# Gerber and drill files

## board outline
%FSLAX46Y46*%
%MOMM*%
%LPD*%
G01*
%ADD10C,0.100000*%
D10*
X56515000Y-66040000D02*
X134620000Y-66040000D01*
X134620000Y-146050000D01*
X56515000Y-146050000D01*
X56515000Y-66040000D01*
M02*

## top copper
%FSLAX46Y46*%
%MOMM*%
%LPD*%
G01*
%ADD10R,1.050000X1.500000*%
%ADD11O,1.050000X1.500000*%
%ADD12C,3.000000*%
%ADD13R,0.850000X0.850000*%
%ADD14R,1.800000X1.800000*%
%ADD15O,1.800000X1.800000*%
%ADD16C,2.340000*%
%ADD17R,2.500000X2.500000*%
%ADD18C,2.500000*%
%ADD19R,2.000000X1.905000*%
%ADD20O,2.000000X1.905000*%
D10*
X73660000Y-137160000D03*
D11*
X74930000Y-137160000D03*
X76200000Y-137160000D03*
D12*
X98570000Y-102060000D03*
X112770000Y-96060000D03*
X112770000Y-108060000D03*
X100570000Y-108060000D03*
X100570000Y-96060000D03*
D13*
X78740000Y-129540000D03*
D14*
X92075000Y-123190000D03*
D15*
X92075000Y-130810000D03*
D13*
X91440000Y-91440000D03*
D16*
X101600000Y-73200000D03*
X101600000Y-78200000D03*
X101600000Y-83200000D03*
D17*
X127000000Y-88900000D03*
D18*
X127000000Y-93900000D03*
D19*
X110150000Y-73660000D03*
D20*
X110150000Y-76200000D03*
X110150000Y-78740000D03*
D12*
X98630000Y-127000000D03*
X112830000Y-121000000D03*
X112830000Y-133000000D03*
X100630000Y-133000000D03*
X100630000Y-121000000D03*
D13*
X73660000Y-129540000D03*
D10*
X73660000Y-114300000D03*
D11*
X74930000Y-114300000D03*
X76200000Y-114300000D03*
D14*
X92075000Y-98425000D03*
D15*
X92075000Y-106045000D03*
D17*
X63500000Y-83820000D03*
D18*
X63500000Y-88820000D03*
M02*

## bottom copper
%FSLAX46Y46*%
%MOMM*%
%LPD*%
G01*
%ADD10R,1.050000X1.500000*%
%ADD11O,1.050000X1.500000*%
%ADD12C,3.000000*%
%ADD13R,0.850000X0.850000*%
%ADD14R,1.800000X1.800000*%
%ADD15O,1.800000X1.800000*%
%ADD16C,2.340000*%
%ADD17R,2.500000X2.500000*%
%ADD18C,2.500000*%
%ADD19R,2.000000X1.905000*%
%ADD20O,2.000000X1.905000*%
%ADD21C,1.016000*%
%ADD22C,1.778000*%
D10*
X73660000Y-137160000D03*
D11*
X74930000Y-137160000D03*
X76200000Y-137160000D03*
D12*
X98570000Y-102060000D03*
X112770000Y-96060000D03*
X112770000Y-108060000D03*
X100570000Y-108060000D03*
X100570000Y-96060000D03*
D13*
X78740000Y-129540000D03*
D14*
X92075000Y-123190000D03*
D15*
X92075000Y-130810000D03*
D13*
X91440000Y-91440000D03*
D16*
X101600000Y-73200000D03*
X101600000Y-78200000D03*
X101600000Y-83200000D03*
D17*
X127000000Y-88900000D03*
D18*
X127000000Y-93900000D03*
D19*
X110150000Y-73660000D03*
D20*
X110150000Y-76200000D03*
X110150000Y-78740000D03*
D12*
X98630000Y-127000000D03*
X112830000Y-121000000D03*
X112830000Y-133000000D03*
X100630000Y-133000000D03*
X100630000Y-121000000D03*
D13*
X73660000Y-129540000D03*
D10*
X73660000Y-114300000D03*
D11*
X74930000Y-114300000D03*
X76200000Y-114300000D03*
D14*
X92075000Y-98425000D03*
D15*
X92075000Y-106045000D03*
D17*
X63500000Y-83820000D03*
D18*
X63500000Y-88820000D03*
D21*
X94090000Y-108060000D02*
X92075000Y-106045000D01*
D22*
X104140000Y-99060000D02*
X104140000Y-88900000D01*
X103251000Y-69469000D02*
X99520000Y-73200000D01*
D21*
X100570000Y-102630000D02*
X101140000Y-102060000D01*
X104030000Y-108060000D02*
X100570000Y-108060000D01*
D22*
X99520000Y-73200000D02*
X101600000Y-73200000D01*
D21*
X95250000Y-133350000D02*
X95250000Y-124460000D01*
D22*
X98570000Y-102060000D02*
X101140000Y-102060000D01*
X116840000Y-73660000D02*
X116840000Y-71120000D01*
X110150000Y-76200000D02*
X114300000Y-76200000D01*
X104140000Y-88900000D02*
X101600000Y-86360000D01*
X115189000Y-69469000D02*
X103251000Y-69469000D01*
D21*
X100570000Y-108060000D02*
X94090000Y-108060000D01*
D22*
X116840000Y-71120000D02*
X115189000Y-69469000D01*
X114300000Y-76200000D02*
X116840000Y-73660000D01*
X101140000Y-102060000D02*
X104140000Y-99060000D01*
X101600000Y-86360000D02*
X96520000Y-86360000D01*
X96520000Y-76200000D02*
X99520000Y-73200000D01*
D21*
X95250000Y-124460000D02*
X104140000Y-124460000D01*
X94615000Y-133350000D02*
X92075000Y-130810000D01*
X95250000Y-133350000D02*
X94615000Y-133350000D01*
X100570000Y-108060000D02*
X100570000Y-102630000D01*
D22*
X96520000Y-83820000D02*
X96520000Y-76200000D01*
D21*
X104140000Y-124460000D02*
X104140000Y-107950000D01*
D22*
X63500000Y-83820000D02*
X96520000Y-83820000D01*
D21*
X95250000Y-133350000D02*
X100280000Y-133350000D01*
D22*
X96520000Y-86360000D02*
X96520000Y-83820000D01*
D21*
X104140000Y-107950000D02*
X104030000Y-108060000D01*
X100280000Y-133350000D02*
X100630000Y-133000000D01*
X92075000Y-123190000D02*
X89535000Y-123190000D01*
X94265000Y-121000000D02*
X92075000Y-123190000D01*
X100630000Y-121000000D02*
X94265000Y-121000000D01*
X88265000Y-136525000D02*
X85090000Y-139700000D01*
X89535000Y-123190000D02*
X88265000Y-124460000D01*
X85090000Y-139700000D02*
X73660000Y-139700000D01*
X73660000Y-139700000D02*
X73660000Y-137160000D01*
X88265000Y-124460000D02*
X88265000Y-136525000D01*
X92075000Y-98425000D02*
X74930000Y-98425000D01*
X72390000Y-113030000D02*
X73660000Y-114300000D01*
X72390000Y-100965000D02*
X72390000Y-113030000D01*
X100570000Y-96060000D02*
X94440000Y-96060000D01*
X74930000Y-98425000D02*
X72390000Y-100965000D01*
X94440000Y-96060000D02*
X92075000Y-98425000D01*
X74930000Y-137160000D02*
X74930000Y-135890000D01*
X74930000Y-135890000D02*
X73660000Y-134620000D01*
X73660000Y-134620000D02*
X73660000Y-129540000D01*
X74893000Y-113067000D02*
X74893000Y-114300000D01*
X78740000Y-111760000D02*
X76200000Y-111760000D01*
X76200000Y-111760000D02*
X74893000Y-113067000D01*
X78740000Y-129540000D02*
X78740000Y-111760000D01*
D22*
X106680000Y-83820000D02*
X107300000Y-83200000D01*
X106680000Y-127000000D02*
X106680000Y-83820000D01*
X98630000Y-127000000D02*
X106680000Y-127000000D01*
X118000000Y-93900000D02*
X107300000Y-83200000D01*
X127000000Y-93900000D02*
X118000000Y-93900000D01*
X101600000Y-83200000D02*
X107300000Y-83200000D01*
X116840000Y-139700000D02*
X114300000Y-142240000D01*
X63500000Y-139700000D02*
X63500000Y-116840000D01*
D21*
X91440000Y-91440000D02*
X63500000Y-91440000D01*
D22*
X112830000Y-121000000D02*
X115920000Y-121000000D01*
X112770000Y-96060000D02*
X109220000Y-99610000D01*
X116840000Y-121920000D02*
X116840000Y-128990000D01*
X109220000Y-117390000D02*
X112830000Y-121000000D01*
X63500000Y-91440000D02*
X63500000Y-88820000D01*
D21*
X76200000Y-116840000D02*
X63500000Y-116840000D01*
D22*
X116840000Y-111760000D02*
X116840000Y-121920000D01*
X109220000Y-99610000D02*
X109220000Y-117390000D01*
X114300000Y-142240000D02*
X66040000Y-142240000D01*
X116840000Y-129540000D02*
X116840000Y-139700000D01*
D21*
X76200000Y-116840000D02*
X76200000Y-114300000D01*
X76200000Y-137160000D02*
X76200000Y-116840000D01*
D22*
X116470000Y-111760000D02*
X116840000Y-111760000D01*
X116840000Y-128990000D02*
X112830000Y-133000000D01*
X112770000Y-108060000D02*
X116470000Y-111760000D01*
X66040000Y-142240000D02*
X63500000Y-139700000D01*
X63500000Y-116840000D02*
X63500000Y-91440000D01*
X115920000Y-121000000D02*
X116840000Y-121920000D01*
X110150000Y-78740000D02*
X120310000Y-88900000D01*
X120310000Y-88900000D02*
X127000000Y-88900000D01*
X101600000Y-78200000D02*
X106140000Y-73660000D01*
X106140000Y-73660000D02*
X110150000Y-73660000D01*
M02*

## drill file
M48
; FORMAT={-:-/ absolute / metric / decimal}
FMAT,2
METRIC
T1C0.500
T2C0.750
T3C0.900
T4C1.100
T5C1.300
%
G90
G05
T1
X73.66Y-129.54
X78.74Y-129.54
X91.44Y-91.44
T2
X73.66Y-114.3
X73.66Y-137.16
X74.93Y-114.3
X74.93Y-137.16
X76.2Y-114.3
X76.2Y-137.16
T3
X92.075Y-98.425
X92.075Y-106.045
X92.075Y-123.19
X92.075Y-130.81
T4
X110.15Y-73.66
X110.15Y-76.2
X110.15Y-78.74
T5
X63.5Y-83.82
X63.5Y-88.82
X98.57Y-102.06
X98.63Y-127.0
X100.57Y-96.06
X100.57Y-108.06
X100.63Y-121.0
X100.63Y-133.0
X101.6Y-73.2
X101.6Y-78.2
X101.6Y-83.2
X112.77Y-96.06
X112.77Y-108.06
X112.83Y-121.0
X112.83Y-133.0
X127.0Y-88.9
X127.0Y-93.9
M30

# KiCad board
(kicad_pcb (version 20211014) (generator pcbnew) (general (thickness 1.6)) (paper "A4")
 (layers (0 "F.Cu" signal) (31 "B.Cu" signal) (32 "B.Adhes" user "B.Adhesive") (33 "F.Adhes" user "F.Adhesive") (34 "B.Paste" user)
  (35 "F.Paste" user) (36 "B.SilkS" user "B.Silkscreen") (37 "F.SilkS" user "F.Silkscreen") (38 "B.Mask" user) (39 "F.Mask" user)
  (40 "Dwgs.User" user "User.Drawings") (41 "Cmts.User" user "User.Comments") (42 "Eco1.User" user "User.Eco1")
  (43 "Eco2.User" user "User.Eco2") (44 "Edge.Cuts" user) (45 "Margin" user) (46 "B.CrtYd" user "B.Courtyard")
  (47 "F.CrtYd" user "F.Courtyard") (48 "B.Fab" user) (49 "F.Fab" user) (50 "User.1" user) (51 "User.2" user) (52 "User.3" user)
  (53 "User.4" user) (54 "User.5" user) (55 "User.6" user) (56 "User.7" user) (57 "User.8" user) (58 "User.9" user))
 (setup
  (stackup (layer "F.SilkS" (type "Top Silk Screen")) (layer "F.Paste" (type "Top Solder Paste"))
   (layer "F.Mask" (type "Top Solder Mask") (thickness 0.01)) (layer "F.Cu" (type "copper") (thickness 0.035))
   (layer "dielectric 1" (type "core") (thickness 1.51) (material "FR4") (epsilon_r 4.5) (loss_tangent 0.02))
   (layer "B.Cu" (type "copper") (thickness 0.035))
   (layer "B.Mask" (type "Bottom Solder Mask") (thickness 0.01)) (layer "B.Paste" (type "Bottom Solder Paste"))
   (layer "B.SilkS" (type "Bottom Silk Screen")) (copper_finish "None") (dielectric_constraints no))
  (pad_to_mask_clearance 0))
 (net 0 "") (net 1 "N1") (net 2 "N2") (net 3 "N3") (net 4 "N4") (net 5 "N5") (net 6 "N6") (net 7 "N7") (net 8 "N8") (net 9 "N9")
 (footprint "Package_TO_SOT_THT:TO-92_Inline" (layer "F.Cu") (at 73.66 137.16)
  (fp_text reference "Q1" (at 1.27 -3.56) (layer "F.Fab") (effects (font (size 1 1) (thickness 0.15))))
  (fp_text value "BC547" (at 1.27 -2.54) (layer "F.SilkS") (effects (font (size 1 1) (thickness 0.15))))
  (pad "1" thru_hole rect (at 0 0) (size 1.05 1.5) (drill 0.75) (layers *.Cu *.Mask) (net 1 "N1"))
  (pad "2" thru_hole oval (at 1.27 0) (size 1.05 1.5) (drill 0.75) (layers *.Cu *.Mask) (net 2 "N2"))
  (pad "3" thru_hole oval (at 2.54 0) (size 1.05 1.5) (drill 0.75) (layers *.Cu *.Mask) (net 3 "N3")))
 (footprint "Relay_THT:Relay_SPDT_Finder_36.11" (layer "F.Cu") (at 98.57 102.06)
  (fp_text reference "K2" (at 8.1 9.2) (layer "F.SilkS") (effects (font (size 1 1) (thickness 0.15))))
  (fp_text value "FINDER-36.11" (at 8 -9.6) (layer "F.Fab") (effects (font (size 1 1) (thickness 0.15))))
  (pad "11" thru_hole circle (at 0 0) (size 3 3) (drill 1.3) (layers *.Cu *.Mask) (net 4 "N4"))
  (pad "12" thru_hole circle (at 14.2 -6) (size 3 3) (drill 1.3) (layers *.Cu *.Mask) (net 3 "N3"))
  (pad "14" thru_hole circle (at 14.2 6) (size 3 3) (drill 1.3) (layers *.Cu *.Mask) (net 3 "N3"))
  (pad "A1" thru_hole circle (at 2 6) (size 3 3) (drill 1.3) (layers *.Cu *.Mask) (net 4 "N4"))
  (pad "A2" thru_hole circle (at 2 -6) (size 3 3) (drill 1.3) (layers *.Cu *.Mask) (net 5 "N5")))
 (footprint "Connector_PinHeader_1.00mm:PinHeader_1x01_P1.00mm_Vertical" (layer "F.Cu") (at 78.74 129.54)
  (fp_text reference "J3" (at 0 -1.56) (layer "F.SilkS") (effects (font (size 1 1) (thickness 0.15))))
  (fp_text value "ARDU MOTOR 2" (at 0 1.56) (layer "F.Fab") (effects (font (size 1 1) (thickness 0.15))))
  (pad "1" thru_hole rect (at 0 0) (size 0.85 0.85) (drill 0.5) (layers *.Cu *.Mask) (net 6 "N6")))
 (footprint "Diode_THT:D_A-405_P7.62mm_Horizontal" (layer "F.Cu") (at 92.075 123.19 -90)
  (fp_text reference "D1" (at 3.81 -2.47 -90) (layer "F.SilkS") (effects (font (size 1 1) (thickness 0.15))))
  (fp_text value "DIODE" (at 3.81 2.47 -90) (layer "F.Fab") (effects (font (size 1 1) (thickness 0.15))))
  (pad "1" thru_hole rect (at 0 0 270) (size 1.8 1.8) (drill 0.9) (layers *.Cu *.Mask) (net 1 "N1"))
  (pad "2" thru_hole oval (at 7.62 0 270) (size 1.8 1.8) (drill 0.9) (layers *.Cu *.Mask) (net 4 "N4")))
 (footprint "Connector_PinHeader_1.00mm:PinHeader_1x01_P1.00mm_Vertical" (layer "F.Cu") (at 91.44 91.44)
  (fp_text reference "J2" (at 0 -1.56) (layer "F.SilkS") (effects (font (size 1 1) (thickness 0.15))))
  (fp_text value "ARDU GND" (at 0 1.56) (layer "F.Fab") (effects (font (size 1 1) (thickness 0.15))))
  (pad "1" thru_hole rect (at 0 0) (size 0.85 0.85) (drill 0.5) (layers *.Cu *.Mask) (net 3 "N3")))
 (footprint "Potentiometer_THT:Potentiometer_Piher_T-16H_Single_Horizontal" (layer "F.Cu") (at 101.6 73.2 180)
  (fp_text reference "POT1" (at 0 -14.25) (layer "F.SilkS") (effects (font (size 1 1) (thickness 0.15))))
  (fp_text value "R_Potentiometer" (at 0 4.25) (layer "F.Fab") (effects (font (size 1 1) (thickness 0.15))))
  (pad "1" thru_hole circle (at 0 0 180) (size 2.34 2.34) (drill 1.3) (layers *.Cu *.Mask) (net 4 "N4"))
  (pad "2" thru_hole circle (at 0 -5 180) (size 2.34 2.34) (drill 1.3) (layers *.Cu *.Mask) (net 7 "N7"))
  (pad "3" thru_hole circle (at 0 -10 180) (size 2.34 2.34) (drill 1.3) (layers *.Cu *.Mask) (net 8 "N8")))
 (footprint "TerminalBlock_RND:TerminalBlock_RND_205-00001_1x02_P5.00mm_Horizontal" (layer "F.Cu") (at 127 88.9 -90)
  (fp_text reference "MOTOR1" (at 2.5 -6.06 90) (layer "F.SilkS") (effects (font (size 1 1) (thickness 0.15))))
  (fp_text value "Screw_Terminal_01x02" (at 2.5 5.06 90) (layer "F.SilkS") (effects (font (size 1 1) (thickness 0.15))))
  (pad "1" thru_hole rect (at 0 0 270) (size 2.5 2.5) (drill 1.3) (layers *.Cu *.Mask) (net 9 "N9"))
  (pad "2" thru_hole circle (at 5 0 270) (size 2.5 2.5) (drill 1.3) (layers *.Cu *.Mask) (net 8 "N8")))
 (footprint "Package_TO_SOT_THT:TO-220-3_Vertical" (layer "F.Cu") (at 110.15 73.66 -90)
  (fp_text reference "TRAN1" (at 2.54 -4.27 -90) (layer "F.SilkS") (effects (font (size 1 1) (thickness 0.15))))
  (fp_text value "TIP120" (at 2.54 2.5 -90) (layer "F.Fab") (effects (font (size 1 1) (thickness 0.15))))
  (pad "1" thru_hole rect (at 0 0 270) (size 1.905 2) (drill 1.1) (layers *.Cu *.Mask) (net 7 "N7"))
  (pad "2" thru_hole oval (at 2.54 0 270) (size 1.905 2) (drill 1.1) (layers *.Cu *.Mask) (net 4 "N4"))
  (pad "3" thru_hole oval (at 5.08 0 270) (size 1.905 2) (drill 1.1) (layers *.Cu *.Mask) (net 9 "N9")))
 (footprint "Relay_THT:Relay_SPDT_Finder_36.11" (layer "F.Cu") (at 98.63 127)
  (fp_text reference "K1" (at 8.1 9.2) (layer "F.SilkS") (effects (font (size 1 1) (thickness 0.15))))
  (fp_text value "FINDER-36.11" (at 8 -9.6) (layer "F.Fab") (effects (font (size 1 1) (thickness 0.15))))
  (pad "11" thru_hole circle (at 0 0) (size 3 3) (drill 1.3) (layers *.Cu *.Mask) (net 8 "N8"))
  (pad "12" thru_hole circle (at 14.2 -6) (size 3 3) (drill 1.3) (layers *.Cu *.Mask) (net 3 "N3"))
  (pad "14" thru_hole circle (at 14.2 6) (size 3 3) (drill 1.3) (layers *.Cu *.Mask) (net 3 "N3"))
  (pad "A1" thru_hole circle (at 2 6) (size 3 3) (drill 1.3) (layers *.Cu *.Mask) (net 4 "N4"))
  (pad "A2" thru_hole circle (at 2 -6) (size 3 3) (drill 1.3) (layers *.Cu *.Mask) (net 1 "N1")))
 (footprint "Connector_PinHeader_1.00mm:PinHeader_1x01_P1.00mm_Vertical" (layer "F.Cu") (at 73.66 129.54)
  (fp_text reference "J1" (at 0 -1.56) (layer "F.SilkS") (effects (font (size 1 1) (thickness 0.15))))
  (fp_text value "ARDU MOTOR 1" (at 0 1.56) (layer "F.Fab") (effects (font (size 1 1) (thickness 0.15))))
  (pad "1" thru_hole rect (at 0 0) (size 0.85 0.85) (drill 0.5) (layers *.Cu *.Mask) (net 2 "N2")))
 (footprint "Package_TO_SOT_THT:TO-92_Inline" (layer "F.Cu") (at 73.66 114.3)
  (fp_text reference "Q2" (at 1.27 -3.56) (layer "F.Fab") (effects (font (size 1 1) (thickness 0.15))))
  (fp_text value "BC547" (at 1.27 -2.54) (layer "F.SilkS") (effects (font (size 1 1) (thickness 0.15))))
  (pad "1" thru_hole rect (at 0 0) (size 1.05 1.5) (drill 0.75) (layers *.Cu *.Mask) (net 5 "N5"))
  (pad "2" thru_hole oval (at 1.27 0) (size 1.05 1.5) (drill 0.75) (layers *.Cu *.Mask) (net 6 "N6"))
  (pad "3" thru_hole oval (at 2.54 0) (size 1.05 1.5) (drill 0.75) (layers *.Cu *.Mask) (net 3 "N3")))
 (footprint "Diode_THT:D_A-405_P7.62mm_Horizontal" (layer "F.Cu") (at 92.075 98.425 -90)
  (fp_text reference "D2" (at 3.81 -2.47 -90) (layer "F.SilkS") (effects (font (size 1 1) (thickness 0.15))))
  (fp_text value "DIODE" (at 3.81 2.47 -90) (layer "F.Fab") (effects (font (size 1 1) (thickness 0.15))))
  (pad "1" thru_hole rect (at 0 0 270) (size 1.8 1.8) (drill 0.9) (layers *.Cu *.Mask) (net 5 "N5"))
  (pad "2" thru_hole oval (at 7.62 0 270) (size 1.8 1.8) (drill 0.9) (layers *.Cu *.Mask) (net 4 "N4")))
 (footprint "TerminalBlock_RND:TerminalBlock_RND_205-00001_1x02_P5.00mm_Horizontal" (layer "F.Cu") (at 63.5 83.82 -90)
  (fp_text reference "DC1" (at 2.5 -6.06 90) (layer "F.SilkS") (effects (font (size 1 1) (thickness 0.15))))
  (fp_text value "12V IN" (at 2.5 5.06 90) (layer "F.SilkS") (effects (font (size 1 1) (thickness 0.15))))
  (pad "1" thru_hole rect (at 0 0 270) (size 2.5 2.5) (drill 1.3) (layers *.Cu *.Mask) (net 4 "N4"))
  (pad "2" thru_hole circle (at 5 0 270) (size 2.5 2.5) (drill 1.3) (layers *.Cu *.Mask) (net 3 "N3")))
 (gr_rect (start 56.515 146.05) (end 134.62 66.04) (layer "Edge.Cuts") (width 0.1) (fill none))
 (segment (start 94.09 108.06) (end 92.075 106.045) (width 1.016) (layer "B.Cu") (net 4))
 (segment (start 104.14 99.06) (end 104.14 88.9) (width 1.778) (layer "B.Cu") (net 4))
 (segment (start 103.251 69.469) (end 99.52 73.2) (width 1.778) (layer "B.Cu") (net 4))
 (segment (start 100.57 102.63) (end 101.14 102.06) (width 1.016) (layer "B.Cu") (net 4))
 (segment (start 104.03 108.06) (end 100.57 108.06) (width 1.016) (layer "B.Cu") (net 4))
 (segment (start 99.52 73.2) (end 101.6 73.2) (width 1.778) (layer "B.Cu") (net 4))
 (segment (start 95.25 133.35) (end 95.25 124.46) (width 1.016) (layer "B.Cu") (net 4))
 (segment (start 98.57 102.06) (end 101.14 102.06) (width 1.778) (layer "B.Cu") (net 4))
 (segment (start 116.84 73.66) (end 116.84 71.12) (width 1.778) (layer "B.Cu") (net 4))
 (segment (start 110.15 76.2) (end 114.3 76.2) (width 1.778) (layer "B.Cu") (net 4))
 (segment (start 104.14 88.9) (end 101.6 86.36) (width 1.778) (layer "B.Cu") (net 4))
 (segment (start 115.189 69.469) (end 103.251 69.469) (width 1.778) (layer "B.Cu") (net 4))
 (segment (start 100.57 108.06) (end 94.09 108.06) (width 1.016) (layer "B.Cu") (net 4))
 (segment (start 116.84 71.12) (end 115.189 69.469) (width 1.778) (layer "B.Cu") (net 4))
 (segment (start 114.3 76.2) (end 116.84 73.66) (width 1.778) (layer "B.Cu") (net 4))
 (segment (start 101.14 102.06) (end 104.14 99.06) (width 1.778) (layer "B.Cu") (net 4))
 (segment (start 101.6 86.36) (end 96.52 86.36) (width 1.778) (layer "B.Cu") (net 4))
 (segment (start 96.52 76.2) (end 99.52 73.2) (width 1.778) (layer "B.Cu") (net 4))
 (segment (start 95.25 124.46) (end 104.14 124.46) (width 1.016) (layer "B.Cu") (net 4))
 (segment (start 94.615 133.35) (end 92.075 130.81) (width 1.016) (layer "B.Cu") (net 4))
 (segment (start 95.25 133.35) (end 94.615 133.35) (width 1.016) (layer "B.Cu") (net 4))
 (segment (start 100.57 108.06) (end 100.57 102.63) (width 1.016) (layer "B.Cu") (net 4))
 (segment (start 96.52 83.82) (end 96.52 76.2) (width 1.778) (layer "B.Cu") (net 4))
 (segment (start 104.14 124.46) (end 104.14 107.95) (width 1.016) (layer "B.Cu") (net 4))
 (segment (start 63.5 83.82) (end 96.52 83.82) (width 1.778) (layer "B.Cu") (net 4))
 (segment (start 95.25 133.35) (end 100.28 133.35) (width 1.016) (layer "B.Cu") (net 4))
 (segment (start 96.52 86.36) (end 96.52 83.82) (width 1.778) (layer "B.Cu") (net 4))
 (segment (start 104.14 107.95) (end 104.03 108.06) (width 1.016) (layer "B.Cu") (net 4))
 (segment (start 100.28 133.35) (end 100.63 133) (width 1.016) (layer "B.Cu") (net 4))
 (segment (start 92.075 123.19) (end 89.535 123.19) (width 1.016) (layer "B.Cu") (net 1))
 (segment (start 94.265 121) (end 92.075 123.19) (width 1.016) (layer "B.Cu") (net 1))
 (segment (start 100.63 121) (end 94.265 121) (width 1.016) (layer "B.Cu") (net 1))
 (segment (start 88.265 136.525) (end 85.09 139.7) (width 1.016) (layer "B.Cu") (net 1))
 (segment (start 89.535 123.19) (end 88.265 124.46) (width 1.016) (layer "B.Cu") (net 1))
 (segment (start 85.09 139.7) (end 73.66 139.7) (width 1.016) (layer "B.Cu") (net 1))
 (segment (start 73.66 139.7) (end 73.66 137.16) (width 1.016) (layer "B.Cu") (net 1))
 (segment (start 88.265 124.46) (end 88.265 136.525) (width 1.016) (layer "B.Cu") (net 1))
 (segment (start 92.075 98.425) (end 74.93 98.425) (width 1.016) (layer "B.Cu") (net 5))
 (segment (start 72.39 113.03) (end 73.66 114.3) (width 1.016) (layer "B.Cu") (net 5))
 (segment (start 72.39 100.965) (end 72.39 113.03) (width 1.016) (layer "B.Cu") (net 5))
 (segment (start 100.57 96.06) (end 94.44 96.06) (width 1.016) (layer "B.Cu") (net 5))
 (segment (start 74.93 98.425) (end 72.39 100.965) (width 1.016) (layer "B.Cu") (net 5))
 (segment (start 94.44 96.06) (end 92.075 98.425) (width 1.016) (layer "B.Cu") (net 5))
 (segment (start 74.93 137.16) (end 74.93 135.89) (width 1.016) (layer "B.Cu") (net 2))
 (segment (start 74.93 135.89) (end 73.66 134.62) (width 1.016) (layer "B.Cu") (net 2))
 (segment (start 73.66 134.62) (end 73.66 129.54) (width 1.016) (layer "B.Cu") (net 2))
 (segment (start 74.893 113.067) (end 74.893 114.3) (width 1.016) (layer "B.Cu") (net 6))
 (segment (start 78.74 111.76) (end 76.2 111.76) (width 1.016) (layer "B.Cu") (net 6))
 (segment (start 76.2 111.76) (end 74.893 113.067) (width 1.016) (layer "B.Cu") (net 6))
 (segment (start 78.74 129.54) (end 78.74 111.76) (width 1.016) (layer "B.Cu") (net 6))
 (segment (start 106.68 83.82) (end 107.3 83.2) (width 1.778) (layer "B.Cu") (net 8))
 (segment (start 106.68 127) (end 106.68 83.82) (width 1.778) (layer "B.Cu") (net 8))
 (segment (start 98.63 127) (end 106.68 127) (width 1.778) (layer "B.Cu") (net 8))
 (segment (start 118 93.9) (end 107.3 83.2) (width 1.778) (layer "B.Cu") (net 8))
 (segment (start 127 93.9) (end 118 93.9) (width 1.778) (layer "B.Cu") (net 8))
 (segment (start 101.6 83.2) (end 107.3 83.2) (width 1.778) (layer "B.Cu") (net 8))
 (segment (start 116.84 139.7) (end 114.3 142.24) (width 1.778) (layer "B.Cu") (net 3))
 (segment (start 63.5 139.7) (end 63.5 116.84) (width 1.778) (layer "B.Cu") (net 3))
 (segment (start 91.44 91.44) (end 63.5 91.44) (width 1.016) (layer "B.Cu") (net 3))
 (segment (start 112.83 121) (end 115.92 121) (width 1.778) (layer "B.Cu") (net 3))
 (segment (start 112.77 96.06) (end 109.22 99.61) (width 1.778) (layer "B.Cu") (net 3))
 (segment (start 116.84 121.92) (end 116.84 128.99) (width 1.778) (layer "B.Cu") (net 3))
 (segment (start 109.22 117.39) (end 112.83 121) (width 1.778) (layer "B.Cu") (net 3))
 (segment (start 63.5 91.44) (end 63.5 88.82) (width 1.778) (layer "B.Cu") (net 3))
 (segment (start 76.2 116.84) (end 63.5 116.84) (width 1.016) (layer "B.Cu") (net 3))
 (segment (start 116.84 111.76) (end 116.84 121.92) (width 1.778) (layer "B.Cu") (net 3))
 (segment (start 109.22 99.61) (end 109.22 117.39) (width 1.778) (layer "B.Cu") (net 3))
 (segment (start 114.3 142.24) (end 66.04 142.24) (width 1.778) (layer "B.Cu") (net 3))
 (segment (start 116.84 129.54) (end 116.84 139.7) (width 1.778) (layer "B.Cu") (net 3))
 (segment (start 76.2 116.84) (end 76.2 114.3) (width 1.016) (layer "B.Cu") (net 3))
 (segment (start 76.2 137.16) (end 76.2 116.84) (width 1.016) (layer "B.Cu") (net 3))
 (segment (start 116.47 111.76) (end 116.84 111.76) (width 1.778) (layer "B.Cu") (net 3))
 (segment (start 116.84 128.99) (end 112.83 133) (width 1.778) (layer "B.Cu") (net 3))
 (segment (start 112.77 108.06) (end 116.47 111.76) (width 1.778) (layer "B.Cu") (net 3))
 (segment (start 66.04 142.24) (end 63.5 139.7) (width 1.778) (layer "B.Cu") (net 3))
 (segment (start 63.5 116.84) (end 63.5 91.44) (width 1.778) (layer "B.Cu") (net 3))
 (segment (start 115.92 121) (end 116.84 121.92) (width 1.778) (layer "B.Cu") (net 3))
 (segment (start 110.15 78.74) (end 120.31 88.9) (width 1.778) (layer "B.Cu") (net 9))
 (segment (start 120.31 88.9) (end 127 88.9) (width 1.778) (layer "B.Cu") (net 9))
 (segment (start 101.6 78.2) (end 106.14 73.66) (width 1.778) (layer "B.Cu") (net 7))
 (segment (start 106.14 73.66) (end 110.15 73.66) (width 1.778) (layer "B.Cu") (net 7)))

